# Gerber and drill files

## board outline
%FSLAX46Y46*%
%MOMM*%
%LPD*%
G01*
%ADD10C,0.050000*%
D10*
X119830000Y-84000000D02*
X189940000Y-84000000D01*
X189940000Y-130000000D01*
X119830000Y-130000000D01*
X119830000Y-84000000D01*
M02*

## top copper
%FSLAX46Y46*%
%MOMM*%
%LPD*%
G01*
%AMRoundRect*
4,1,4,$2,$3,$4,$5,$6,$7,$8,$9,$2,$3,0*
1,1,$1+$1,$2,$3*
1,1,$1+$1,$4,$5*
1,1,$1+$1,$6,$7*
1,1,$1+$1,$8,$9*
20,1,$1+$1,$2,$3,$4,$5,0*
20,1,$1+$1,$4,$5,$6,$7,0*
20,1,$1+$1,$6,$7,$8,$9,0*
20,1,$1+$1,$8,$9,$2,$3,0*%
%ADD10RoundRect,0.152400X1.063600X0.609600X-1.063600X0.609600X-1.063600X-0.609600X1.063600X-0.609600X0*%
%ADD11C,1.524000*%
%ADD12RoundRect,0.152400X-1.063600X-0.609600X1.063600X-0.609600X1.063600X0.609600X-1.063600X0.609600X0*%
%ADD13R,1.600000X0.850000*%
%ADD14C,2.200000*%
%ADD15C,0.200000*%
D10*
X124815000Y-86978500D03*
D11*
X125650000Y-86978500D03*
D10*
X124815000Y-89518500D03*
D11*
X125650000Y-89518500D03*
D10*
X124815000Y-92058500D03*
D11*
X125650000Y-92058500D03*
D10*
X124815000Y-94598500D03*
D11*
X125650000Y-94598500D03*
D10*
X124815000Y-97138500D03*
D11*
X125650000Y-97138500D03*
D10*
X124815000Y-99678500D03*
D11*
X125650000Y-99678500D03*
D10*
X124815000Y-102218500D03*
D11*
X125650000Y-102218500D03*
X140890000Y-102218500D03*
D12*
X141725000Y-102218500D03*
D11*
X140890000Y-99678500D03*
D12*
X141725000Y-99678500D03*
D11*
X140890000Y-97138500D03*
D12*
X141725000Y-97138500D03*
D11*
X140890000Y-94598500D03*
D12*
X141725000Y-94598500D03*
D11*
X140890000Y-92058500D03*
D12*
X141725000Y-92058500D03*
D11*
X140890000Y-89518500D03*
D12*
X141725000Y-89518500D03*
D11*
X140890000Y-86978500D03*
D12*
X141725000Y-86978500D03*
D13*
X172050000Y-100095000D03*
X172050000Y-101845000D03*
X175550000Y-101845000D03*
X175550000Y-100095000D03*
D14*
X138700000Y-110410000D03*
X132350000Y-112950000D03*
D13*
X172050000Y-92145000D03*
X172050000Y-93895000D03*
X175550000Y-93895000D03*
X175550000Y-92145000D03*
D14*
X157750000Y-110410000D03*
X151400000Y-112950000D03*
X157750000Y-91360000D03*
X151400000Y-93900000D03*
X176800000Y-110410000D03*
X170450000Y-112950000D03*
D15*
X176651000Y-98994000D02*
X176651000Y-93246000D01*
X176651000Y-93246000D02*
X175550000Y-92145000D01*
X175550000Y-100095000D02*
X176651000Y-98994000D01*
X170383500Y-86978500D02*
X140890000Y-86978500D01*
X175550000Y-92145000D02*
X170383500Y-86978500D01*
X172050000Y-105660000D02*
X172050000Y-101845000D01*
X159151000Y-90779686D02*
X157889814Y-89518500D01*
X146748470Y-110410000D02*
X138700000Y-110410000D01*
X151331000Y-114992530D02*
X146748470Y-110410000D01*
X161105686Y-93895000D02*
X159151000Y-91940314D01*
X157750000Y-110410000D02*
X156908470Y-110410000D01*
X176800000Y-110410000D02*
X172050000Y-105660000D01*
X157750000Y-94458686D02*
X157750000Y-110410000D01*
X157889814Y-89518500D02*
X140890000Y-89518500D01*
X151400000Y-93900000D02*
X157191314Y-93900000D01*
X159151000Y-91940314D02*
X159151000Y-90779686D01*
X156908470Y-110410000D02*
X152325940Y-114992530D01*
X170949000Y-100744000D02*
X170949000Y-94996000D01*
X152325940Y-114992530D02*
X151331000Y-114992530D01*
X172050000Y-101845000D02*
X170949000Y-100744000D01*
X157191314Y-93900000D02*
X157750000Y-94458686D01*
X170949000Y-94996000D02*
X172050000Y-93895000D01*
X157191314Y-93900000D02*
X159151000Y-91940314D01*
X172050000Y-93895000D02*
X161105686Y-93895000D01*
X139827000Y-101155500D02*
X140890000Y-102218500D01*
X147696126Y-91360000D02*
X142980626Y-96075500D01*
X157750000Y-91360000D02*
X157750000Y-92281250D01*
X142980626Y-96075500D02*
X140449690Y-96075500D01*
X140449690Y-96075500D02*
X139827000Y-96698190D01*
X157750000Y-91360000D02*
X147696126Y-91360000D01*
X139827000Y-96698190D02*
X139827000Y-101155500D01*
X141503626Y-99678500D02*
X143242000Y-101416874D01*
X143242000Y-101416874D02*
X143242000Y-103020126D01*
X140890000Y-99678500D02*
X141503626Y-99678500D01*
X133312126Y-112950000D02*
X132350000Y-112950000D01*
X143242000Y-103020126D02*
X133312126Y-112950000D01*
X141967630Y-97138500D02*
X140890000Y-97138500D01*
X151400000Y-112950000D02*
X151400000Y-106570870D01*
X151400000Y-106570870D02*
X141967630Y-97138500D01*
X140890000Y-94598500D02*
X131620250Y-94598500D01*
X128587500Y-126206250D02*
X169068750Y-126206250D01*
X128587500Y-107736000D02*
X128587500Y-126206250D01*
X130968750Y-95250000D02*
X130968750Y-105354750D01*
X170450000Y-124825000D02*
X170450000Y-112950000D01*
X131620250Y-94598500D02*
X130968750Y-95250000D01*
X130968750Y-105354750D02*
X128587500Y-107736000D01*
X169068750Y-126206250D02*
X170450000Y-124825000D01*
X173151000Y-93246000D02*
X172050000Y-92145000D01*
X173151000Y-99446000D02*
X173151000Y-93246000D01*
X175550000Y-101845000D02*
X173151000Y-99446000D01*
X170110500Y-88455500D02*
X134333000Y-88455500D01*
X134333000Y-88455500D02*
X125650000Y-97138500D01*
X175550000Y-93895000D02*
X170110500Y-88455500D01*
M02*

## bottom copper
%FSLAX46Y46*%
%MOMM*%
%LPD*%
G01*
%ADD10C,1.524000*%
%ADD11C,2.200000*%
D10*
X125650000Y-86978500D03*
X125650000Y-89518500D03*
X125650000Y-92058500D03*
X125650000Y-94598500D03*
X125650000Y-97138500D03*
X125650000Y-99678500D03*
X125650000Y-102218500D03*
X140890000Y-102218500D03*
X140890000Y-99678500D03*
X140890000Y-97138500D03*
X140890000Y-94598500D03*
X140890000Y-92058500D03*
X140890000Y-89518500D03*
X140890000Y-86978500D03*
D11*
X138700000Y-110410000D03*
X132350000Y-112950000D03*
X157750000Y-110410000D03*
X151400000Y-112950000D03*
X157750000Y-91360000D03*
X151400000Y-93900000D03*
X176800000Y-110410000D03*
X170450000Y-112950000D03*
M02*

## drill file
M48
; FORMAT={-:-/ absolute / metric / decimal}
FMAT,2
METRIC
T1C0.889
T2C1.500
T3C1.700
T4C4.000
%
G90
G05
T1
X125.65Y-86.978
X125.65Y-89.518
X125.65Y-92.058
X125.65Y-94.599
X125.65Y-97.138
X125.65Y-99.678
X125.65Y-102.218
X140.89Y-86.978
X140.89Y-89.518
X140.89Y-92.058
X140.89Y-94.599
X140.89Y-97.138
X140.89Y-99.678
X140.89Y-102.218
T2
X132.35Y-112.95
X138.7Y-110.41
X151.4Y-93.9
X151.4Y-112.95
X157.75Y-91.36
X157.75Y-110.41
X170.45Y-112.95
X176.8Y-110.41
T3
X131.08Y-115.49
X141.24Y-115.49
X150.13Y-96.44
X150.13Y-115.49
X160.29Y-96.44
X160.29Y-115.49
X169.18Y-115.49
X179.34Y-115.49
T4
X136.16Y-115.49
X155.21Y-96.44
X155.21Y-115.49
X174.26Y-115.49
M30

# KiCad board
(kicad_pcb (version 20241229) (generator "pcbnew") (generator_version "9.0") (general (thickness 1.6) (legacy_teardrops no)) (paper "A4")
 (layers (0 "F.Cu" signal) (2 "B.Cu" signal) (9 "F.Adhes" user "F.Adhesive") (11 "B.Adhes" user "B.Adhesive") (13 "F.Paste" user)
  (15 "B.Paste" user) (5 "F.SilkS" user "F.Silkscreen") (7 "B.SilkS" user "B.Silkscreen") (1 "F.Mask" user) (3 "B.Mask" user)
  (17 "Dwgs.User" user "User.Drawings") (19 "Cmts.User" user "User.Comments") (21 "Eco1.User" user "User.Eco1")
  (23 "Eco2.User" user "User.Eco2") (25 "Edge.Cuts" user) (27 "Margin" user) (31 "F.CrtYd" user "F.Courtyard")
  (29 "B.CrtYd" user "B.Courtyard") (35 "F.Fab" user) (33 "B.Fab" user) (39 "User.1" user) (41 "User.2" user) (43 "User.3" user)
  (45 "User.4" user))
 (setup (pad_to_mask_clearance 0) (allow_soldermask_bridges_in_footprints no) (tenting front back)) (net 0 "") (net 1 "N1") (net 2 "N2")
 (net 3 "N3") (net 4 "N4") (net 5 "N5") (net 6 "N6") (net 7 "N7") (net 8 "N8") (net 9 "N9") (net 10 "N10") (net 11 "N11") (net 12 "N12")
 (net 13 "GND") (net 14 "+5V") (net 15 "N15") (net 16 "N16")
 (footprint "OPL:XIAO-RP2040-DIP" (layer "F.Cu") (at 133.27 94.5985)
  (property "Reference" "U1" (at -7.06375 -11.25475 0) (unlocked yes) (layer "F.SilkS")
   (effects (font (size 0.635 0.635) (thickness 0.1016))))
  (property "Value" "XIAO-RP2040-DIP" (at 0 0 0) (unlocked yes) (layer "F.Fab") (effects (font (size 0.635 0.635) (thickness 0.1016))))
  (pad "1" smd roundrect (at -8.455 -7.62 180) (size 2.432 1.524) (layers "F.Cu" "F.Mask") (roundrect_rratio 0.1) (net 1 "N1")
   (thermal_bridge_angle 45))
  (pad "1" thru_hole circle (at -7.62 -7.62 180) (size 1.524 1.524) (drill 0.889) (layers "*.Cu" "*.Mask") (remove_unused_layers no)
   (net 1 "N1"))
  (pad "2" smd roundrect (at -8.455 -5.08 180) (size 2.432 1.524) (layers "F.Cu" "F.Mask") (roundrect_rratio 0.1) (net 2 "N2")
   (thermal_bridge_angle 45))
  (pad "2" thru_hole circle (at -7.62 -5.08 180) (size 1.524 1.524) (drill 0.889) (layers "*.Cu" "*.Mask") (remove_unused_layers no)
   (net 2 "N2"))
  (pad "3" smd roundrect (at -8.455 -2.54 180) (size 2.432 1.524) (layers "F.Cu" "F.Mask") (roundrect_rratio 0.1) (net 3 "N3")
   (thermal_bridge_angle 45))
  (pad "3" thru_hole circle (at -7.62 -2.54 180) (size 1.524 1.524) (drill 0.889) (layers "*.Cu" "*.Mask") (remove_unused_layers no)
   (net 3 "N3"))
  (pad "4" smd roundrect (at -8.455 0 180) (size 2.432 1.524) (layers "F.Cu" "F.Mask") (roundrect_rratio 0.1) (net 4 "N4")
   (thermal_bridge_angle 45))
  (pad "4" thru_hole circle (at -7.62 0 180) (size 1.524 1.524) (drill 0.889) (layers "*.Cu" "*.Mask") (remove_unused_layers no)
   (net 4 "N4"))
  (pad "5" smd roundrect (at -8.455 2.54 180) (size 2.432 1.524) (layers "F.Cu" "F.Mask") (roundrect_rratio 0.1) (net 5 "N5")
   (thermal_bridge_angle 45))
  (pad "5" thru_hole circle (at -7.62 2.54 180) (size 1.524 1.524) (drill 0.889) (layers "*.Cu" "*.Mask") (remove_unused_layers no)
   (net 5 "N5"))
  (pad "6" smd roundrect (at -8.455 5.08 180) (size 2.432 1.524) (layers "F.Cu" "F.Mask") (roundrect_rratio 0.1) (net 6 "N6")
   (thermal_bridge_angle 45))
  (pad "6" thru_hole circle (at -7.62 5.08 180) (size 1.524 1.524) (drill 0.889) (layers "*.Cu" "*.Mask") (remove_unused_layers no)
   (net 6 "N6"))
  (pad "7" smd roundrect (at -8.455 7.62 180) (size 2.432 1.524) (layers "F.Cu" "F.Mask") (roundrect_rratio 0.1) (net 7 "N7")
   (thermal_bridge_angle 45))
  (pad "7" thru_hole circle (at -7.62 7.62 180) (size 1.524 1.524) (drill 0.889) (layers "*.Cu" "*.Mask") (remove_unused_layers no)
   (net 7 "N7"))
  (pad "8" thru_hole circle (at 7.62 7.62) (size 1.524 1.524) (drill 0.889) (layers "*.Cu" "*.Mask") (remove_unused_layers no) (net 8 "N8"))
  (pad "8" smd roundrect (at 8.455 7.62) (size 2.432 1.524) (layers "F.Cu" "F.Mask") (roundrect_rratio 0.1) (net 8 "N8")
   (thermal_bridge_angle 45))
  (pad "9" thru_hole circle (at 7.62 5.08) (size 1.524 1.524) (drill 0.889) (layers "*.Cu" "*.Mask") (remove_unused_layers no) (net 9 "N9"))
  (pad "9" smd roundrect (at 8.455 5.08) (size 2.432 1.524) (layers "F.Cu" "F.Mask") (roundrect_rratio 0.1) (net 9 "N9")
   (thermal_bridge_angle 45))
  (pad "10" thru_hole circle (at 7.62 2.54) (size 1.524 1.524) (drill 0.889) (layers "*.Cu" "*.Mask") (remove_unused_layers no)
   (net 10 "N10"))
  (pad "10" smd roundrect (at 8.455 2.54) (size 2.432 1.524) (layers "F.Cu" "F.Mask") (roundrect_rratio 0.1) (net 10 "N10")
   (thermal_bridge_angle 45))
  (pad "11" thru_hole circle (at 7.62 0) (size 1.524 1.524) (drill 0.889) (layers "*.Cu" "*.Mask") (remove_unused_layers no) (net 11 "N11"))
  (pad "11" smd roundrect (at 8.455 0) (size 2.432 1.524) (layers "F.Cu" "F.Mask") (roundrect_rratio 0.1) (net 11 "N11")
   (thermal_bridge_angle 45))
  (pad "12" thru_hole circle (at 7.62 -2.54) (size 1.524 1.524) (drill 0.889) (layers "*.Cu" "*.Mask") (remove_unused_layers no)
   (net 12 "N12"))
  (pad "12" smd roundrect (at 8.455 -2.54) (size 2.432 1.524) (layers "F.Cu" "F.Mask") (roundrect_rratio 0.1) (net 12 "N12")
   (thermal_bridge_angle 45))
  (pad "13" thru_hole circle (at 7.62 -5.08) (size 1.524 1.524) (drill 0.889) (layers "*.Cu" "*.Mask") (remove_unused_layers no)
   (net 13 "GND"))
  (pad "13" smd roundrect (at 8.455 -5.08) (size 2.432 1.524) (layers "F.Cu" "F.Mask") (roundrect_rratio 0.1) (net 13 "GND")
   (thermal_bridge_angle 45))
  (pad "14" thru_hole circle (at 7.62 -7.62) (size 1.524 1.524) (drill 0.889) (layers "*.Cu" "*.Mask") (remove_unused_layers no)
   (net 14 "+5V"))
  (pad "14" smd roundrect (at 8.455 -7.62) (size 2.432 1.524) (layers "F.Cu" "F.Mask") (roundrect_rratio 0.1) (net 14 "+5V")
   (thermal_bridge_angle 45)))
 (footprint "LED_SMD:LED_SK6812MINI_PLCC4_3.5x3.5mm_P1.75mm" (layer "F.Cu") (at 173.8 100.97)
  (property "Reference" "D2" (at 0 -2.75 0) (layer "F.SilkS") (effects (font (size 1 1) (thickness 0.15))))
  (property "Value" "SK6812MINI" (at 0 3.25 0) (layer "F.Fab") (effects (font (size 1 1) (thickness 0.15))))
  (pad "1" smd rect (at -1.75 -0.875) (size 1.6 0.85) (layers "F.Cu" "F.Mask" "F.Paste") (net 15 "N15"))
  (pad "2" smd rect (at -1.75 0.875) (size 1.6 0.85) (layers "F.Cu" "F.Mask" "F.Paste") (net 13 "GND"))
  (pad "3" smd rect (at 1.75 0.875) (size 1.6 0.85) (layers "F.Cu" "F.Mask" "F.Paste") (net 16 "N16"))
  (pad "4" smd rect (at 1.75 -0.875) (size 1.6 0.85) (layers "F.Cu" "F.Mask" "F.Paste") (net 14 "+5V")))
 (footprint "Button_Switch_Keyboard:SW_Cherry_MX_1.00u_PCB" (layer "F.Cu") (at 138.7 110.41)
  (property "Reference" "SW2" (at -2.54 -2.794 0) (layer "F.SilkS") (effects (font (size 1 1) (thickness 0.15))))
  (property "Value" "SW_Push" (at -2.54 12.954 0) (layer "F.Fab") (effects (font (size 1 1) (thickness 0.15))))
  (pad "" np_thru_hole circle (at -7.62 5.08) (size 1.7 1.7) (drill 1.7) (layers "*.Cu" "*.Mask"))
  (pad "" np_thru_hole circle (at -2.54 5.08) (size 4 4) (drill 4) (layers "*.Cu" "*.Mask"))
  (pad "" np_thru_hole circle (at 2.54 5.08) (size 1.7 1.7) (drill 1.7) (layers "*.Cu" "*.Mask"))
  (pad "1" thru_hole circle (at 0 0) (size 2.2 2.2) (drill 1.5) (layers "*.Cu" "*.Mask") (remove_unused_layers no) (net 13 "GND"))
  (pad "2" thru_hole circle (at -6.35 2.54) (size 2.2 2.2) (drill 1.5) (layers "*.Cu" "*.Mask") (remove_unused_layers no) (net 9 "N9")))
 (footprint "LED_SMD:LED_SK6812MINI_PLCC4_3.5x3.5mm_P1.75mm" (layer "F.Cu") (at 173.8 93.02)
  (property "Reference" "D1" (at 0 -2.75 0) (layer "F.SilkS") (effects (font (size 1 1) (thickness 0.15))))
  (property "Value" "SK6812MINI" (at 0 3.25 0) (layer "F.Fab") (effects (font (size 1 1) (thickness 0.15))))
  (pad "1" smd rect (at -1.75 -0.875) (size 1.6 0.85) (layers "F.Cu" "F.Mask" "F.Paste") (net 16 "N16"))
  (pad "2" smd rect (at -1.75 0.875) (size 1.6 0.85) (layers "F.Cu" "F.Mask" "F.Paste") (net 13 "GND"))
  (pad "3" smd rect (at 1.75 0.875) (size 1.6 0.85) (layers "F.Cu" "F.Mask" "F.Paste") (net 5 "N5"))
  (pad "4" smd rect (at 1.75 -0.875) (size 1.6 0.85) (layers "F.Cu" "F.Mask" "F.Paste") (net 14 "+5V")))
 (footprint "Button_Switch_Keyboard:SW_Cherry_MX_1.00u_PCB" (layer "F.Cu") (at 157.75 110.41)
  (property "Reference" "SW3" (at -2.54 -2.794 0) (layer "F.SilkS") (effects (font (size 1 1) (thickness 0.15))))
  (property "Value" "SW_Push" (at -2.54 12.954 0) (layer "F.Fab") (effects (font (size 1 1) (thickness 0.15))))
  (pad "" np_thru_hole circle (at -7.62 5.08) (size 1.7 1.7) (drill 1.7) (layers "*.Cu" "*.Mask"))
  (pad "" np_thru_hole circle (at -2.54 5.08) (size 4 4) (drill 4) (layers "*.Cu" "*.Mask"))
  (pad "" np_thru_hole circle (at 2.54 5.08) (size 1.7 1.7) (drill 1.7) (layers "*.Cu" "*.Mask"))
  (pad "1" thru_hole circle (at 0 0) (size 2.2 2.2) (drill 1.5) (layers "*.Cu" "*.Mask") (remove_unused_layers no) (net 13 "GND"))
  (pad "2" thru_hole circle (at -6.35 2.54) (size 2.2 2.2) (drill 1.5) (layers "*.Cu" "*.Mask") (remove_unused_layers no) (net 10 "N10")))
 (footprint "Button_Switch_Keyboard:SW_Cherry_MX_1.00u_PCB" (layer "F.Cu") (at 157.75 91.36)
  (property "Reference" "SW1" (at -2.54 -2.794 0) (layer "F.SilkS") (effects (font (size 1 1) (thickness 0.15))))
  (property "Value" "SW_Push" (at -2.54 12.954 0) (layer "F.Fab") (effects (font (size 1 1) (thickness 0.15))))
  (pad "" np_thru_hole circle (at -7.62 5.08) (size 1.7 1.7) (drill 1.7) (layers "*.Cu" "*.Mask"))
  (pad "" np_thru_hole circle (at -2.54 5.08) (size 4 4) (drill 4) (layers "*.Cu" "*.Mask"))
  (pad "" np_thru_hole circle (at 2.54 5.08) (size 1.7 1.7) (drill 1.7) (layers "*.Cu" "*.Mask"))
  (pad "1" thru_hole circle (at 0 0) (size 2.2 2.2) (drill 1.5) (layers "*.Cu" "*.Mask") (remove_unused_layers no) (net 8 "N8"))
  (pad "2" thru_hole circle (at -6.35 2.54) (size 2.2 2.2) (drill 1.5) (layers "*.Cu" "*.Mask") (remove_unused_layers no) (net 13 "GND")))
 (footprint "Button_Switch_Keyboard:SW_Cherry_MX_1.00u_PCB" (layer "F.Cu") (at 176.8 110.41)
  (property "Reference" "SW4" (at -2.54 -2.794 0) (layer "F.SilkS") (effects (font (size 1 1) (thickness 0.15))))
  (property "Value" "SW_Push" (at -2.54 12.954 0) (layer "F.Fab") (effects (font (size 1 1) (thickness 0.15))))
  (pad "" np_thru_hole circle (at -7.62 5.08) (size 1.7 1.7) (drill 1.7) (layers "*.Cu" "*.Mask"))
  (pad "" np_thru_hole circle (at -2.54 5.08) (size 4 4) (drill 4) (layers "*.Cu" "*.Mask"))
  (pad "" np_thru_hole circle (at 2.54 5.08) (size 1.7 1.7) (drill 1.7) (layers "*.Cu" "*.Mask"))
  (pad "1" thru_hole circle (at 0 0) (size 2.2 2.2) (drill 1.5) (layers "*.Cu" "*.Mask") (remove_unused_layers no) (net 13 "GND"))
  (pad "2" thru_hole circle (at -6.35 2.54) (size 2.2 2.2) (drill 1.5) (layers "*.Cu" "*.Mask") (remove_unused_layers no) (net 11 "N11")))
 (gr_rect (start 119.83 84) (end 189.94 130) (stroke (width 0.05) (type default)) (fill no) (layer "Edge.Cuts"))
 (segment (start 176.651 98.994) (end 176.651 93.246) (width 0.2) (layer "F.Cu") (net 14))
 (segment (start 176.651 93.246) (end 175.55 92.145) (width 0.2) (layer "F.Cu") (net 14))
 (segment (start 175.55 100.095) (end 176.651 98.994) (width 0.2) (layer "F.Cu") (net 14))
 (segment (start 170.3835 86.9785) (end 140.89 86.9785) (width 0.2) (layer "F.Cu") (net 14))
 (segment (start 175.55 92.145) (end 170.3835 86.9785) (width 0.2) (layer "F.Cu") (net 14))
 (segment (start 172.05 105.66) (end 172.05 101.845) (width 0.2) (layer "F.Cu") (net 13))
 (segment (start 159.151 90.779686) (end 157.889814 89.5185) (width 0.2) (layer "F.Cu") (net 13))
 (segment (start 146.74847 110.41) (end 138.7 110.41) (width 0.2) (layer "F.Cu") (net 13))
 (segment (start 151.331 114.99253) (end 146.74847 110.41) (width 0.2) (layer "F.Cu") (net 13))
 (segment (start 161.105686 93.895) (end 159.151 91.940314) (width 0.2) (layer "F.Cu") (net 13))
 (segment (start 157.75 110.41) (end 156.90847 110.41) (width 0.2) (layer "F.Cu") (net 13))
 (segment (start 176.8 110.41) (end 172.05 105.66) (width 0.2) (layer "F.Cu") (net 13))
 (segment (start 157.75 94.458686) (end 157.75 110.41) (width 0.2) (layer "F.Cu") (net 13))
 (segment (start 157.889814 89.5185) (end 140.89 89.5185) (width 0.2) (layer "F.Cu") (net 13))
 (segment (start 151.4 93.9) (end 157.191314 93.9) (width 0.2) (layer "F.Cu") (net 13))
 (segment (start 159.151 91.940314) (end 159.151 90.779686) (width 0.2) (layer "F.Cu") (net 13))
 (segment (start 156.90847 110.41) (end 152.32594 114.99253) (width 0.2) (layer "F.Cu") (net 13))
 (segment (start 170.949 100.744) (end 170.949 94.996) (width 0.2) (layer "F.Cu") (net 13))
 (segment (start 152.32594 114.99253) (end 151.331 114.99253) (width 0.2) (layer "F.Cu") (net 13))
 (segment (start 172.05 101.845) (end 170.949 100.744) (width 0.2) (layer "F.Cu") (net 13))
 (segment (start 157.191314 93.9) (end 157.75 94.458686) (width 0.2) (layer "F.Cu") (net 13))
 (segment (start 170.949 94.996) (end 172.05 93.895) (width 0.2) (layer "F.Cu") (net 13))
 (segment (start 157.191314 93.9) (end 159.151 91.940314) (width 0.2) (layer "F.Cu") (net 13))
 (segment (start 172.05 93.895) (end 161.105686 93.895) (width 0.2) (layer "F.Cu") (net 13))
 (segment (start 139.827 101.1555) (end 140.89 102.2185) (width 0.2) (layer "F.Cu") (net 8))
 (segment (start 147.696126 91.36) (end 142.980626 96.0755) (width 0.2) (layer "F.Cu") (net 8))
 (segment (start 157.75 91.36) (end 157.75 92.28125) (width 0.2) (layer "F.Cu") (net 8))
 (segment (start 142.980626 96.0755) (end 140.44969 96.0755) (width 0.2) (layer "F.Cu") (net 8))
 (segment (start 140.44969 96.0755) (end 139.827 96.69819) (width 0.2) (layer "F.Cu") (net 8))
 (segment (start 157.75 91.36) (end 147.696126 91.36) (width 0.2) (layer "F.Cu") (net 8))
 (segment (start 139.827 96.69819) (end 139.827 101.1555) (width 0.2) (layer "F.Cu") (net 8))
 (segment (start 141.503626 99.6785) (end 143.242 101.416874) (width 0.2) (layer "F.Cu") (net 9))
 (segment (start 143.242 101.416874) (end 143.242 103.020126) (width 0.2) (layer "F.Cu") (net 9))
 (segment (start 140.89 99.6785) (end 141.503626 99.6785) (width 0.2) (layer "F.Cu") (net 9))
 (segment (start 133.312126 112.95) (end 132.35 112.95) (width 0.2) (layer "F.Cu") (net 9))
 (segment (start 143.242 103.020126) (end 133.312126 112.95) (width 0.2) (layer "F.Cu") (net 9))
 (segment (start 141.96763 97.1385) (end 140.89 97.1385) (width 0.2) (layer "F.Cu") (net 10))
 (segment (start 151.4 112.95) (end 151.4 106.57087) (width 0.2) (layer "F.Cu") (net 10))
 (segment (start 151.4 106.57087) (end 141.96763 97.1385) (width 0.2) (layer "F.Cu") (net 10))
 (segment (start 140.89 94.5985) (end 131.62025 94.5985) (width 0.2) (layer "F.Cu") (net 11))
 (segment (start 128.5875 126.20625) (end 169.06875 126.20625) (width 0.2) (layer "F.Cu") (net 11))
 (segment (start 128.5875 107.736) (end 128.5875 126.20625) (width 0.2) (layer "F.Cu") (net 11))
 (segment (start 130.96875 95.25) (end 130.96875 105.35475) (width 0.2) (layer "F.Cu") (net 11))
 (segment (start 170.45 124.825) (end 170.45 112.95) (width 0.2) (layer "F.Cu") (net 11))
 (segment (start 131.62025 94.5985) (end 130.96875 95.25) (width 0.2) (layer "F.Cu") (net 11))
 (segment (start 130.96875 105.35475) (end 128.5875 107.736) (width 0.2) (layer "F.Cu") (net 11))
 (segment (start 169.06875 126.20625) (end 170.45 124.825) (width 0.2) (layer "F.Cu") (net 11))
 (segment (start 173.151 93.246) (end 172.05 92.145) (width 0.2) (layer "F.Cu") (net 16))
 (segment (start 173.151 99.446) (end 173.151 93.246) (width 0.2) (layer "F.Cu") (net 16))
 (segment (start 175.55 101.845) (end 173.151 99.446) (width 0.2) (layer "F.Cu") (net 16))
 (segment (start 170.1105 88.4555) (end 134.333 88.4555) (width 0.2) (layer "F.Cu") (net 5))
 (segment (start 134.333 88.4555) (end 125.65 97.1385) (width 0.2) (layer "F.Cu") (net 5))
 (segment (start 175.55 93.895) (end 170.1105 88.4555) (width 0.2) (layer "F.Cu") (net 5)))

